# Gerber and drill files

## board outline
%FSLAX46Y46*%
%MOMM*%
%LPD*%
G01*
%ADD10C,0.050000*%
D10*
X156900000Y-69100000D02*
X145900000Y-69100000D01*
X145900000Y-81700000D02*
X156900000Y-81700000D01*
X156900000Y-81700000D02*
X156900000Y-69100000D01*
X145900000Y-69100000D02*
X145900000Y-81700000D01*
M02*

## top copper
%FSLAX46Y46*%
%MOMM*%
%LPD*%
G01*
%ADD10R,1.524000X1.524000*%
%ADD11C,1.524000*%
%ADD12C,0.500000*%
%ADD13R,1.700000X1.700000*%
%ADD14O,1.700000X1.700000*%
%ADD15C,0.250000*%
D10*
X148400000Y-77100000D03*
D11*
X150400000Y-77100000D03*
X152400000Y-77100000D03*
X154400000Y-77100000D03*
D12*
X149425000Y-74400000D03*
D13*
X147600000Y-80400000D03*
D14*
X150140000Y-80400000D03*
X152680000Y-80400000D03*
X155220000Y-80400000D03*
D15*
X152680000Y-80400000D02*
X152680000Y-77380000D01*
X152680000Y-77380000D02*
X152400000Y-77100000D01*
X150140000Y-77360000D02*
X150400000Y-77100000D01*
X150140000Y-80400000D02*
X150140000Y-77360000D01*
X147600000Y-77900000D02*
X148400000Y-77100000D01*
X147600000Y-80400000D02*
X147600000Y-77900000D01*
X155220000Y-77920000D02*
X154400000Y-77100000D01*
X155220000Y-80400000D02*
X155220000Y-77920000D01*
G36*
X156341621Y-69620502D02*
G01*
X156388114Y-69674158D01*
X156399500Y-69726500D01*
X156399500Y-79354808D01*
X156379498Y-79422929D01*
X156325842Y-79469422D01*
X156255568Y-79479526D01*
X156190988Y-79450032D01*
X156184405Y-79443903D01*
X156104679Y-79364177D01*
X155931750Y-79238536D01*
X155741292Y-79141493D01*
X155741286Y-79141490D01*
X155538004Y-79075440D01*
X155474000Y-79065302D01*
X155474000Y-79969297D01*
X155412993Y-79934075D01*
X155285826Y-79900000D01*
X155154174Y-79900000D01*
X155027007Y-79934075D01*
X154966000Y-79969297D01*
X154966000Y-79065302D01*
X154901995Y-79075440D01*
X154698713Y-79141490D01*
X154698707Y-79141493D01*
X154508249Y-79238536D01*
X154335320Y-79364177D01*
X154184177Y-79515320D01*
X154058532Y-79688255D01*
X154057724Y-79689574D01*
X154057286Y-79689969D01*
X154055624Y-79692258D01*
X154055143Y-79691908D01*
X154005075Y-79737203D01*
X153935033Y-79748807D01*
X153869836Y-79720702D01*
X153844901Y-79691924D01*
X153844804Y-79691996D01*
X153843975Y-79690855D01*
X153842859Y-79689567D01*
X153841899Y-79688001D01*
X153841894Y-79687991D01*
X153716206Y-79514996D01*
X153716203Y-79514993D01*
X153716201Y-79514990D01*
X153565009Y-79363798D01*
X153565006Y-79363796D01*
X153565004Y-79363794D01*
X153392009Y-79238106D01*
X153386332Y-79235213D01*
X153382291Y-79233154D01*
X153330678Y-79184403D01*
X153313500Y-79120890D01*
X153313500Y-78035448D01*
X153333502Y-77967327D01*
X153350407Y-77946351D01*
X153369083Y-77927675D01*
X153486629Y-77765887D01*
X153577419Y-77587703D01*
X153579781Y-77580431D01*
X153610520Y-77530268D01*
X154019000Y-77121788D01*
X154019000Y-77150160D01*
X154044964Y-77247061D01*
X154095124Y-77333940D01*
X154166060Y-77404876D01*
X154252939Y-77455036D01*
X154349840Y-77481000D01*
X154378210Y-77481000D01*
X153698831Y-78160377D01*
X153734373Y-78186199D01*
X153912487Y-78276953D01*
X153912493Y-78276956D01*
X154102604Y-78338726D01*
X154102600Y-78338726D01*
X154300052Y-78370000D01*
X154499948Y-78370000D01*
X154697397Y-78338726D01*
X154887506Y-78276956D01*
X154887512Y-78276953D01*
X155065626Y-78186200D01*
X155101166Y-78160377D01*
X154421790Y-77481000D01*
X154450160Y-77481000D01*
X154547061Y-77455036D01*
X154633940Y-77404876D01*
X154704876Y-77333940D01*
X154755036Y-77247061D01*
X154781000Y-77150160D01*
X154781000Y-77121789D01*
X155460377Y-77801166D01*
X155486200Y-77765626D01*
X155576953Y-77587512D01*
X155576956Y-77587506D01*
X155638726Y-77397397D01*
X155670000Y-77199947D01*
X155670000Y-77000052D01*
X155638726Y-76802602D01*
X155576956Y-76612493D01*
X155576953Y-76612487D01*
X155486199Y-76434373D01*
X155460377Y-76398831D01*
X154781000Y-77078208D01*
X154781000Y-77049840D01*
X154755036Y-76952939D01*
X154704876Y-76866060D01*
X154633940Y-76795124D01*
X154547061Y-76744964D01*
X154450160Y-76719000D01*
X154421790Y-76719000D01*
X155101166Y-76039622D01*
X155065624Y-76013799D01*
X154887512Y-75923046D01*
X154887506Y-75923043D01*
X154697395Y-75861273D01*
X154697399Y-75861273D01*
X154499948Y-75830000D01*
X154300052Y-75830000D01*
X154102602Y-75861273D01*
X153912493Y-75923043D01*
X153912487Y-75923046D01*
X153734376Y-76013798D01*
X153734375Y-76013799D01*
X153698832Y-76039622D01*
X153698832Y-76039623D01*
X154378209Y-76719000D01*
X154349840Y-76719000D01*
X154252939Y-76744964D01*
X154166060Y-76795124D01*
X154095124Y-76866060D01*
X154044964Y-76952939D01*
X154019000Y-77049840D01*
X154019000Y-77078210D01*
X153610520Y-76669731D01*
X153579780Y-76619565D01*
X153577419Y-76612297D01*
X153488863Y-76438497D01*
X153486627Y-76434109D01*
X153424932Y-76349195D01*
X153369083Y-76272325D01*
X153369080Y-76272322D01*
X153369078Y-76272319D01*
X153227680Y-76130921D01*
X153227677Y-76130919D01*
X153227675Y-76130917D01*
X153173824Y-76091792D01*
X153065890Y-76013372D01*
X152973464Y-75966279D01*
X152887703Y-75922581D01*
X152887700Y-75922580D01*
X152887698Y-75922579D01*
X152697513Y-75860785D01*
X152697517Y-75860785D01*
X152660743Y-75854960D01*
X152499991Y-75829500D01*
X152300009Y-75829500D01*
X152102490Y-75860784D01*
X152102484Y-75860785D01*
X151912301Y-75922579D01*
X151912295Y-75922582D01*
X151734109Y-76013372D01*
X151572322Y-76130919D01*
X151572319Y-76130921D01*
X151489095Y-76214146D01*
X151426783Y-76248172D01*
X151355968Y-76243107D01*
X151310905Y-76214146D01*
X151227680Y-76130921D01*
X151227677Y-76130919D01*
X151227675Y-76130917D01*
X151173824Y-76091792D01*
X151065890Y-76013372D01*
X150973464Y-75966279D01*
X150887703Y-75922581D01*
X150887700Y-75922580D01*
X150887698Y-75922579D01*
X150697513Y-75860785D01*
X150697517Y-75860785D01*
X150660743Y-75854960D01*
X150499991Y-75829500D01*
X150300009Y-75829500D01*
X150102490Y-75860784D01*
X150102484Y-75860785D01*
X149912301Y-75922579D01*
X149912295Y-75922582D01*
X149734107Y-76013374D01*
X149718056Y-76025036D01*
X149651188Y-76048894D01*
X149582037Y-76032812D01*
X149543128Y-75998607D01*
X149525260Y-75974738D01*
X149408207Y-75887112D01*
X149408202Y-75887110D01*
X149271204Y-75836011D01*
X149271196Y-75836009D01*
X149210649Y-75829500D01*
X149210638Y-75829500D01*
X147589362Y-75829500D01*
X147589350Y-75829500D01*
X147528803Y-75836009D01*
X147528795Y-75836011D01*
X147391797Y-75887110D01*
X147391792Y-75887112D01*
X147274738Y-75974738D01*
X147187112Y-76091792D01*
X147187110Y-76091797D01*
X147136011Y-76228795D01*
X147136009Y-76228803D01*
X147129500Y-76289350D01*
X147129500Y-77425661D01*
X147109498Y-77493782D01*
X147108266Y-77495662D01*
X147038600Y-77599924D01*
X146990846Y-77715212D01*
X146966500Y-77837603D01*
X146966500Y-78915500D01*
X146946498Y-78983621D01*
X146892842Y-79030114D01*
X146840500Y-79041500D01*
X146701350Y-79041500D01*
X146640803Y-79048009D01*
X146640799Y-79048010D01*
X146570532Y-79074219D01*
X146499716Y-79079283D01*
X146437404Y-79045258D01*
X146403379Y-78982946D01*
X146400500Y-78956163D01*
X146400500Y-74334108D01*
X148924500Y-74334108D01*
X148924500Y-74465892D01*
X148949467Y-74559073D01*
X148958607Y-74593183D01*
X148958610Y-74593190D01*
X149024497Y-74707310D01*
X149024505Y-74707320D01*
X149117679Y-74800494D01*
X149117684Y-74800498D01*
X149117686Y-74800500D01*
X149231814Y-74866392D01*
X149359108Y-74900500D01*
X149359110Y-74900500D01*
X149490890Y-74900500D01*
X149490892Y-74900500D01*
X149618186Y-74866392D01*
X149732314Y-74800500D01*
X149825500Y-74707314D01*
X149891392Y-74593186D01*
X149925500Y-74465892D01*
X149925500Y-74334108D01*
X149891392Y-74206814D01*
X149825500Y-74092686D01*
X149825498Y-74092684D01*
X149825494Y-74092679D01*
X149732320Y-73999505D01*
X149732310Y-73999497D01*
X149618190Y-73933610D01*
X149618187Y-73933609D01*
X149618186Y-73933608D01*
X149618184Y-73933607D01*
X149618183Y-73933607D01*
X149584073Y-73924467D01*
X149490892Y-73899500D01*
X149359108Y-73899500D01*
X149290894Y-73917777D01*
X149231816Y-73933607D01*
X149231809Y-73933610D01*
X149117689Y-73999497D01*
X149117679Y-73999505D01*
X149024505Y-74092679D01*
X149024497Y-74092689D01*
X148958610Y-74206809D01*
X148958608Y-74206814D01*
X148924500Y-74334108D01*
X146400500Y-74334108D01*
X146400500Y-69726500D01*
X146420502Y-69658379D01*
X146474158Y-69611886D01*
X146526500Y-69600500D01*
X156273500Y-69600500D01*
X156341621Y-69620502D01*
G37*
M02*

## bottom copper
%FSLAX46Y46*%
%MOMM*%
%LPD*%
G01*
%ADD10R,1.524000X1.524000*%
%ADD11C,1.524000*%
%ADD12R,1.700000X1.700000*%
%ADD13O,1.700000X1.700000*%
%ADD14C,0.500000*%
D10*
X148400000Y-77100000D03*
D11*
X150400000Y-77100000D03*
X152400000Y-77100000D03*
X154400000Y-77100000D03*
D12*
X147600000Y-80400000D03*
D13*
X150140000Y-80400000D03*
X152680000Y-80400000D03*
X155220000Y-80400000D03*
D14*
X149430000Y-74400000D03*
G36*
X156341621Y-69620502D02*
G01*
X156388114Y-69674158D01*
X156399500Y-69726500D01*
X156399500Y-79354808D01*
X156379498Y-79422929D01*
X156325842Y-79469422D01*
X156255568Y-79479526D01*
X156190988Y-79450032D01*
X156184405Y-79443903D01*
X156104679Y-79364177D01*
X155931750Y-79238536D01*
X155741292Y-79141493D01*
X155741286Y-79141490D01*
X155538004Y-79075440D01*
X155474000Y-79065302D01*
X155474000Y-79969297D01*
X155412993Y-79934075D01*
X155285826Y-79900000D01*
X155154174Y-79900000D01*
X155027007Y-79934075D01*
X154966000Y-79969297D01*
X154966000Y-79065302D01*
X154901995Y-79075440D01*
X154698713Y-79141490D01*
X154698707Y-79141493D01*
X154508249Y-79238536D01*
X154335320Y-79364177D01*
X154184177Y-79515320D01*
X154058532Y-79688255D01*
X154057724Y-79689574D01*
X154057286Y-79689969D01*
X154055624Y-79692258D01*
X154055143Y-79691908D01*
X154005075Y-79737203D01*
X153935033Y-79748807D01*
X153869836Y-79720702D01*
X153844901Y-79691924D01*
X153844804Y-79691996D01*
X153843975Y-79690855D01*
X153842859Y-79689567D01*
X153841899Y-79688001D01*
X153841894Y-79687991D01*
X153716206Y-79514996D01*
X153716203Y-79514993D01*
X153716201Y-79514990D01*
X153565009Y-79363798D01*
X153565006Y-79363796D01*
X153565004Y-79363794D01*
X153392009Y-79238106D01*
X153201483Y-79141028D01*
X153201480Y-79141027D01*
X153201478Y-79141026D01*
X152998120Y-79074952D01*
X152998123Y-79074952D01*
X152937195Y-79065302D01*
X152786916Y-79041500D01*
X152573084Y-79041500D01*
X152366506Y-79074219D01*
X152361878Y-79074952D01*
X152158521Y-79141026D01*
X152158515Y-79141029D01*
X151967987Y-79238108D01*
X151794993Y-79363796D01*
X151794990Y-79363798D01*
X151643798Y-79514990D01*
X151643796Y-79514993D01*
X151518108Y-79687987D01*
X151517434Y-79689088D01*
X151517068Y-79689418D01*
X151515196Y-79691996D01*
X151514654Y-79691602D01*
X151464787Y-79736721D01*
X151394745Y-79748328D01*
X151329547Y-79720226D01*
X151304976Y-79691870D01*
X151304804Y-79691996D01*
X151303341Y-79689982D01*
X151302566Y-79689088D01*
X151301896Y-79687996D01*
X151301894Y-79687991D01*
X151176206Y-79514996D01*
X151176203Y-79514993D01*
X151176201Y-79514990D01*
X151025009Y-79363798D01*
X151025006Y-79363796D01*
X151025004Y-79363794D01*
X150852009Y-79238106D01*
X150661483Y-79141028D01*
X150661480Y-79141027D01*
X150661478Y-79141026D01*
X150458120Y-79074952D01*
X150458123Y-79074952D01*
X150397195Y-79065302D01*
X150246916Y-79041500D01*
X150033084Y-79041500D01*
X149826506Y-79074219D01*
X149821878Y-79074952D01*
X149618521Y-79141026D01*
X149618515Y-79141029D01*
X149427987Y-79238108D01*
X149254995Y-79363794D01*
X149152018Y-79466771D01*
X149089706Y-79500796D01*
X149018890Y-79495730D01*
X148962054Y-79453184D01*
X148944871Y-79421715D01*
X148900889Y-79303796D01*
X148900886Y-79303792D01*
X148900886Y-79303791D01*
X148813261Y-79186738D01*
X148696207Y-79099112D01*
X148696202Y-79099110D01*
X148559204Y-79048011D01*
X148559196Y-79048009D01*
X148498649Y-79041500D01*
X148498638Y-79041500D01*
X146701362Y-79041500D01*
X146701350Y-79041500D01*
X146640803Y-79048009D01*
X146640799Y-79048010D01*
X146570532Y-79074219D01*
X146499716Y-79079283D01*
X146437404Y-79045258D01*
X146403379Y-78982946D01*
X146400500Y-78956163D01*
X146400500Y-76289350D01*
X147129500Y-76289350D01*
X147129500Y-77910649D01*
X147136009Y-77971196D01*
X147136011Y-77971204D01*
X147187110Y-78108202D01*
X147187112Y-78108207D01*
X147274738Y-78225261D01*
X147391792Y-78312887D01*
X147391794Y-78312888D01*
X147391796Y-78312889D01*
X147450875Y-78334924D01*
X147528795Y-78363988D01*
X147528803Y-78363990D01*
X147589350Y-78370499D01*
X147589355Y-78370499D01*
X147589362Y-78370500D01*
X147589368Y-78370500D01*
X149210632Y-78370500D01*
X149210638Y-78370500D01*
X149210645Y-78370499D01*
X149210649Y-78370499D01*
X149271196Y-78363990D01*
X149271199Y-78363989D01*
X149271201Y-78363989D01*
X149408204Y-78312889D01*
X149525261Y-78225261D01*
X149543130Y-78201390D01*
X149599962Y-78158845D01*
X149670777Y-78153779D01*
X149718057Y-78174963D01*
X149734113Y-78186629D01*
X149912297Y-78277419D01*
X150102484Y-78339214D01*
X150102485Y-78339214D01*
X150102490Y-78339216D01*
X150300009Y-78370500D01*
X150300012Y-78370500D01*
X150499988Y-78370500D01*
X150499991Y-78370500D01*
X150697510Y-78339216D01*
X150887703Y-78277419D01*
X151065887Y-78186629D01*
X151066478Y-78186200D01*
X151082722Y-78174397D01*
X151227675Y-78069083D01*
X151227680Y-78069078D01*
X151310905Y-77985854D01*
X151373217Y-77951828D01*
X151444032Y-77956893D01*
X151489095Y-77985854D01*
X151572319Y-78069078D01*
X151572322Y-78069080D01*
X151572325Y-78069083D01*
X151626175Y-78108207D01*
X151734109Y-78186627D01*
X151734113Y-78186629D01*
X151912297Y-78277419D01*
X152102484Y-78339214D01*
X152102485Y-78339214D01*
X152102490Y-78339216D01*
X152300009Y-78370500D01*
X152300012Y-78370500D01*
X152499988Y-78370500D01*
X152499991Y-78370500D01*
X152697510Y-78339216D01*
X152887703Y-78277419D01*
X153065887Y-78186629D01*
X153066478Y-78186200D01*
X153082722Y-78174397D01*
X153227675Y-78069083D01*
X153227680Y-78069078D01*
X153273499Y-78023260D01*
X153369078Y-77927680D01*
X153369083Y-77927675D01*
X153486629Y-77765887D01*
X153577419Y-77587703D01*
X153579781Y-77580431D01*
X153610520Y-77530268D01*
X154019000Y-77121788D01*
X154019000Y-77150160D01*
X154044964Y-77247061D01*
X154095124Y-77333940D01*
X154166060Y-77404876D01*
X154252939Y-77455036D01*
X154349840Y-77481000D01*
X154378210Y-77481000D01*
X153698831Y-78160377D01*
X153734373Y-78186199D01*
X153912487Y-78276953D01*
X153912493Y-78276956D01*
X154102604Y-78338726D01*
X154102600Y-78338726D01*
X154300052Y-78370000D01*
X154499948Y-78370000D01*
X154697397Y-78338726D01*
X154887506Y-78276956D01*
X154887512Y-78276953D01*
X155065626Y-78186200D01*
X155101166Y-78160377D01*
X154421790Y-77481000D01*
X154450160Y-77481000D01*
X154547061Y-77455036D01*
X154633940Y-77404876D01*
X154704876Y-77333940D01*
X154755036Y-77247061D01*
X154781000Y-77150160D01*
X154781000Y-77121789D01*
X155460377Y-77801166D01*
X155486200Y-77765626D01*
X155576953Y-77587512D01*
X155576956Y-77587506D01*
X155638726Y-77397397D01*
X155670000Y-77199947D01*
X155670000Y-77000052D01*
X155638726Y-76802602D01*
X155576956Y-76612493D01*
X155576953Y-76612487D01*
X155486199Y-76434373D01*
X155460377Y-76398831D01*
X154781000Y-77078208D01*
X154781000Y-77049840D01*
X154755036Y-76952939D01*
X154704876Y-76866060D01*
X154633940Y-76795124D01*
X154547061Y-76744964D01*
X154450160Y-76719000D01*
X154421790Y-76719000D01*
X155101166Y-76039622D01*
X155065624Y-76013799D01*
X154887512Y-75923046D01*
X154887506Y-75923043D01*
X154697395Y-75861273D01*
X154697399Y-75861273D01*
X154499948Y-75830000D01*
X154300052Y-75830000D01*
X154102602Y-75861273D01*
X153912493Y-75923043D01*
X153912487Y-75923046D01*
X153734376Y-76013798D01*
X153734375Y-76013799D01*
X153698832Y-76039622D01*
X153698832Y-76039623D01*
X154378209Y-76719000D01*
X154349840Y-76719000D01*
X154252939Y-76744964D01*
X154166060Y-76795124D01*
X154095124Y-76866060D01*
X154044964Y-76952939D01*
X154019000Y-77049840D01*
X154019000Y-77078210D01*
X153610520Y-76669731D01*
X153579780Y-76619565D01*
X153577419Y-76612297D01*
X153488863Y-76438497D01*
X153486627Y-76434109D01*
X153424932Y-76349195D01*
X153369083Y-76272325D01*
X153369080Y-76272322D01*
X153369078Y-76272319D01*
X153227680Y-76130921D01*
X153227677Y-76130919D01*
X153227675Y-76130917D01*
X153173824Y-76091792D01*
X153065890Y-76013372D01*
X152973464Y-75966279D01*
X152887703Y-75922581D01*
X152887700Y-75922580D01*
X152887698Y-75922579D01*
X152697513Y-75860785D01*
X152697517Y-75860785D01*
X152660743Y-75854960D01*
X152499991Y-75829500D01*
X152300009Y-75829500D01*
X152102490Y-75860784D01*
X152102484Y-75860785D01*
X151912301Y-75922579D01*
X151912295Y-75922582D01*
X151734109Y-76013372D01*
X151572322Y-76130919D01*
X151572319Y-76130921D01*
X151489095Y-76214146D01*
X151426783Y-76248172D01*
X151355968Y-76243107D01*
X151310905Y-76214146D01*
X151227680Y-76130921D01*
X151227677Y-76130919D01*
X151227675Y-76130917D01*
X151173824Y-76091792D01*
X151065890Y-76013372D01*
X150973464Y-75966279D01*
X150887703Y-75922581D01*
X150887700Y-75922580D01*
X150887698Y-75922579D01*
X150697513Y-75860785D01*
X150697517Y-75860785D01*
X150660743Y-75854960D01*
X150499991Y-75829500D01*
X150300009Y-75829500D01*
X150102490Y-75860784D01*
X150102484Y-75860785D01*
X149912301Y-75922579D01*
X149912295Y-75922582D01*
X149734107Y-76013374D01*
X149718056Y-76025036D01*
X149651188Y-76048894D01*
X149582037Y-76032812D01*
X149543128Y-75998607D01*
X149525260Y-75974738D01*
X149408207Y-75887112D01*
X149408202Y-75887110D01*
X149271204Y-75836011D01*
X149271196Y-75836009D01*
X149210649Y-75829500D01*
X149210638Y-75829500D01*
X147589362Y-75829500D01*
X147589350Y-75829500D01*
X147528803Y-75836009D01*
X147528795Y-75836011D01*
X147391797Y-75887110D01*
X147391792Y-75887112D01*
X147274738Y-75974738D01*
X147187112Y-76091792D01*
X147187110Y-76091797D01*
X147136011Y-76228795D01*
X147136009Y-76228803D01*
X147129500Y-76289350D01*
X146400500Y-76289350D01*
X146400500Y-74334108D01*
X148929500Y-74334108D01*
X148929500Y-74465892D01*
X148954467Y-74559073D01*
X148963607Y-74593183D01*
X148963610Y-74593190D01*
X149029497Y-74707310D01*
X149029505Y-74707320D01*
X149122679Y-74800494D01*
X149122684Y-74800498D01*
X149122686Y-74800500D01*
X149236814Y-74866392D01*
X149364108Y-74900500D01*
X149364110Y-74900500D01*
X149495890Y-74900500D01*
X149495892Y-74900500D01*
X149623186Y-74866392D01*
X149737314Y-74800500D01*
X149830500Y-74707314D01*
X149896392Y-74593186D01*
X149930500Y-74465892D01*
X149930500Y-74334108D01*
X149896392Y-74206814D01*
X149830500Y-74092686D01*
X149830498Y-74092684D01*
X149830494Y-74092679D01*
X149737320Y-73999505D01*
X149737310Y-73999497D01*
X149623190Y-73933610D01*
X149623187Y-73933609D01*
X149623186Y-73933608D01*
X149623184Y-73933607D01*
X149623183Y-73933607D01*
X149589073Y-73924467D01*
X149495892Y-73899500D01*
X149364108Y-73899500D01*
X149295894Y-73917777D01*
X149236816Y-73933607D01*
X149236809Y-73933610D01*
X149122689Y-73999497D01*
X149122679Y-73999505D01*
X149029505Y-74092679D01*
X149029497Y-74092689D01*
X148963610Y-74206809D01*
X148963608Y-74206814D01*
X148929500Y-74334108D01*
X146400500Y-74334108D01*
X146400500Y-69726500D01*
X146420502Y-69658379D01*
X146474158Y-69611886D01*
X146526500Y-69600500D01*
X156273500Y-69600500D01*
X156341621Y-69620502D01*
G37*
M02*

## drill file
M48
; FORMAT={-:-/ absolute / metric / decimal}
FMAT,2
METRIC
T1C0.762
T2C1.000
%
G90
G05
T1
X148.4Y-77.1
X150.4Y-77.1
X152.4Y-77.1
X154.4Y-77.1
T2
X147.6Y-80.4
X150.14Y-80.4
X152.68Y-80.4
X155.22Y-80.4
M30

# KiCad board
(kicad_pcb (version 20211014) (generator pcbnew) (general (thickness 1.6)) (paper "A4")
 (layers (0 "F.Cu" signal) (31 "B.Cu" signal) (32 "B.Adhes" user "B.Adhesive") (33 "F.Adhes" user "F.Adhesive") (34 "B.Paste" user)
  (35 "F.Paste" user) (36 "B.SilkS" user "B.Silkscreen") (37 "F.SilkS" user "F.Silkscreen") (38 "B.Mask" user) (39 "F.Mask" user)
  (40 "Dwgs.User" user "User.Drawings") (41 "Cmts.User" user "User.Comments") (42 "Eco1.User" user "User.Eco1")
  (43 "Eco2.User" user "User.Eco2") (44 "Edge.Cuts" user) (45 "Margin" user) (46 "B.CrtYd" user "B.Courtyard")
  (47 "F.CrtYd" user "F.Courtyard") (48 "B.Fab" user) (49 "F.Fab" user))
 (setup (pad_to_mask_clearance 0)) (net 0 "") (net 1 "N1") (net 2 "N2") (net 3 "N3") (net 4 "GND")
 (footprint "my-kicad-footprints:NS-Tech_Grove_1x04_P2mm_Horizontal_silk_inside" (layer "F.Cu") (at 151.4 77.1 90)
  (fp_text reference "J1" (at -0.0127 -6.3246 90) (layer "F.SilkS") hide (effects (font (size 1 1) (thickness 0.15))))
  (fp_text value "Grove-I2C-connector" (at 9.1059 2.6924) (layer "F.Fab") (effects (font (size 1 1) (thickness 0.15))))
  (pad "1" thru_hole rect locked (at 0 -3 90) (size 1.524 1.524) (drill 0.762) (layers *.Cu *.Mask) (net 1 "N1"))
  (pad "2" thru_hole circle locked (at 0 -1 90) (size 1.524 1.524) (drill 0.762) (layers *.Cu *.Mask) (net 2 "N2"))
  (pad "3" thru_hole circle locked (at 0 1 90) (size 1.524 1.524) (drill 0.762) (layers *.Cu *.Mask) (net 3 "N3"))
  (pad "4" thru_hole circle locked (at 0 3 90) (size 1.524 1.524) (drill 0.762) (layers *.Cu *.Mask) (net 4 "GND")))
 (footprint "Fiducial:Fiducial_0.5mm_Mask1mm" (layer "F.Cu") (at 149.425 74.4)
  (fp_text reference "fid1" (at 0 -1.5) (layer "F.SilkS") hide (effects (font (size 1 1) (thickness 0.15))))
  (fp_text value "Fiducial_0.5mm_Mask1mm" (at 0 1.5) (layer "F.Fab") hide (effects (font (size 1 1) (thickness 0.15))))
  (pad "" smd circle locked (at 0 0) (size 0.5 0.5) (layers "F.Cu" "F.Mask") (solder_mask_margin 0.25) (clearance 0.25)))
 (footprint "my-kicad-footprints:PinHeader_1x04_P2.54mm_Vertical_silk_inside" (layer "B.Cu") (at 147.6 80.4 -90)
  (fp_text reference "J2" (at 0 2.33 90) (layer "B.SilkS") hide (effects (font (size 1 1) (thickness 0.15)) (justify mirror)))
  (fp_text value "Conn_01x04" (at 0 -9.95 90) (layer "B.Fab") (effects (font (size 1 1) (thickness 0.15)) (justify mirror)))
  (pad "1" thru_hole rect locked (at 0 0 270) (size 1.7 1.7) (drill 1) (layers *.Cu *.Mask) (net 1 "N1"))
  (pad "2" thru_hole oval locked (at 0 -2.54 270) (size 1.7 1.7) (drill 1) (layers *.Cu *.Mask) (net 2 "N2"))
  (pad "3" thru_hole oval locked (at 0 -5.08 270) (size 1.7 1.7) (drill 1) (layers *.Cu *.Mask) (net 3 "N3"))
  (pad "4" thru_hole oval locked (at 0 -7.62 270) (size 1.7 1.7) (drill 1) (layers *.Cu *.Mask) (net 4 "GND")))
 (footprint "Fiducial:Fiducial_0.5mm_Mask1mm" (layer "B.Cu") (at 149.43 74.4)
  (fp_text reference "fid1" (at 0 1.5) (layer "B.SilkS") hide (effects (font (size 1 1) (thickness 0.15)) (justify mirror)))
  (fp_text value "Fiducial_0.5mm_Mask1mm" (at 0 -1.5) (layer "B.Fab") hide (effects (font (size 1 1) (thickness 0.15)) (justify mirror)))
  (pad "" smd circle locked (at 0 0) (size 0.5 0.5) (layers "B.Cu" "B.Mask") (solder_mask_margin 0.25) (clearance 0.25)))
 (gr_line (start 156.9 69.1) (end 145.9 69.1) (layer "Edge.Cuts") (width 0.05))
 (gr_line (start 145.9 81.7) (end 156.9 81.7) (layer "Edge.Cuts") (width 0.05))
 (gr_line (start 156.9 81.7) (end 156.9 69.1) (layer "Edge.Cuts") (width 0.05))
 (gr_line (start 145.9 69.1) (end 145.9 81.7) (layer "Edge.Cuts") (width 0.05))
 (segment (start 152.68 80.4) (end 152.68 77.38) (width 0.25) (layer "F.Cu") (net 3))
 (segment (start 152.68 77.38) (end 152.4 77.1) (width 0.25) (layer "F.Cu") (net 3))
 (segment (start 150.14 77.36) (end 150.4 77.1) (width 0.25) (layer "F.Cu") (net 2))
 (segment (start 150.14 80.4) (end 150.14 77.36) (width 0.25) (layer "F.Cu") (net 2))
 (segment (start 147.6 77.9) (end 148.4 77.1) (width 0.25) (layer "F.Cu") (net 1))
 (segment (start 147.6 80.4) (end 147.6 77.9) (width 0.25) (layer "F.Cu") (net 1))
 (segment (start 155.22 77.92) (end 154.4 77.1) (width 0.25) (layer "F.Cu") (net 4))
 (segment (start 155.22 80.4) (end 155.22 77.92) (width 0.25) (layer "F.Cu") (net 4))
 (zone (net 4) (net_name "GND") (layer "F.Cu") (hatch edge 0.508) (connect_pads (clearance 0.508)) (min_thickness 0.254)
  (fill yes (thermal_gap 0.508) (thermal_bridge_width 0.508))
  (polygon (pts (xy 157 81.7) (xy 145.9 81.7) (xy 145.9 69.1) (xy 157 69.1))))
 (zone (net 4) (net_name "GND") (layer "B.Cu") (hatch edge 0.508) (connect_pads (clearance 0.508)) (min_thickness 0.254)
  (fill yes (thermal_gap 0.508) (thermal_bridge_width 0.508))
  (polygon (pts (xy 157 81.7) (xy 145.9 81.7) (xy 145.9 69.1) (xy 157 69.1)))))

